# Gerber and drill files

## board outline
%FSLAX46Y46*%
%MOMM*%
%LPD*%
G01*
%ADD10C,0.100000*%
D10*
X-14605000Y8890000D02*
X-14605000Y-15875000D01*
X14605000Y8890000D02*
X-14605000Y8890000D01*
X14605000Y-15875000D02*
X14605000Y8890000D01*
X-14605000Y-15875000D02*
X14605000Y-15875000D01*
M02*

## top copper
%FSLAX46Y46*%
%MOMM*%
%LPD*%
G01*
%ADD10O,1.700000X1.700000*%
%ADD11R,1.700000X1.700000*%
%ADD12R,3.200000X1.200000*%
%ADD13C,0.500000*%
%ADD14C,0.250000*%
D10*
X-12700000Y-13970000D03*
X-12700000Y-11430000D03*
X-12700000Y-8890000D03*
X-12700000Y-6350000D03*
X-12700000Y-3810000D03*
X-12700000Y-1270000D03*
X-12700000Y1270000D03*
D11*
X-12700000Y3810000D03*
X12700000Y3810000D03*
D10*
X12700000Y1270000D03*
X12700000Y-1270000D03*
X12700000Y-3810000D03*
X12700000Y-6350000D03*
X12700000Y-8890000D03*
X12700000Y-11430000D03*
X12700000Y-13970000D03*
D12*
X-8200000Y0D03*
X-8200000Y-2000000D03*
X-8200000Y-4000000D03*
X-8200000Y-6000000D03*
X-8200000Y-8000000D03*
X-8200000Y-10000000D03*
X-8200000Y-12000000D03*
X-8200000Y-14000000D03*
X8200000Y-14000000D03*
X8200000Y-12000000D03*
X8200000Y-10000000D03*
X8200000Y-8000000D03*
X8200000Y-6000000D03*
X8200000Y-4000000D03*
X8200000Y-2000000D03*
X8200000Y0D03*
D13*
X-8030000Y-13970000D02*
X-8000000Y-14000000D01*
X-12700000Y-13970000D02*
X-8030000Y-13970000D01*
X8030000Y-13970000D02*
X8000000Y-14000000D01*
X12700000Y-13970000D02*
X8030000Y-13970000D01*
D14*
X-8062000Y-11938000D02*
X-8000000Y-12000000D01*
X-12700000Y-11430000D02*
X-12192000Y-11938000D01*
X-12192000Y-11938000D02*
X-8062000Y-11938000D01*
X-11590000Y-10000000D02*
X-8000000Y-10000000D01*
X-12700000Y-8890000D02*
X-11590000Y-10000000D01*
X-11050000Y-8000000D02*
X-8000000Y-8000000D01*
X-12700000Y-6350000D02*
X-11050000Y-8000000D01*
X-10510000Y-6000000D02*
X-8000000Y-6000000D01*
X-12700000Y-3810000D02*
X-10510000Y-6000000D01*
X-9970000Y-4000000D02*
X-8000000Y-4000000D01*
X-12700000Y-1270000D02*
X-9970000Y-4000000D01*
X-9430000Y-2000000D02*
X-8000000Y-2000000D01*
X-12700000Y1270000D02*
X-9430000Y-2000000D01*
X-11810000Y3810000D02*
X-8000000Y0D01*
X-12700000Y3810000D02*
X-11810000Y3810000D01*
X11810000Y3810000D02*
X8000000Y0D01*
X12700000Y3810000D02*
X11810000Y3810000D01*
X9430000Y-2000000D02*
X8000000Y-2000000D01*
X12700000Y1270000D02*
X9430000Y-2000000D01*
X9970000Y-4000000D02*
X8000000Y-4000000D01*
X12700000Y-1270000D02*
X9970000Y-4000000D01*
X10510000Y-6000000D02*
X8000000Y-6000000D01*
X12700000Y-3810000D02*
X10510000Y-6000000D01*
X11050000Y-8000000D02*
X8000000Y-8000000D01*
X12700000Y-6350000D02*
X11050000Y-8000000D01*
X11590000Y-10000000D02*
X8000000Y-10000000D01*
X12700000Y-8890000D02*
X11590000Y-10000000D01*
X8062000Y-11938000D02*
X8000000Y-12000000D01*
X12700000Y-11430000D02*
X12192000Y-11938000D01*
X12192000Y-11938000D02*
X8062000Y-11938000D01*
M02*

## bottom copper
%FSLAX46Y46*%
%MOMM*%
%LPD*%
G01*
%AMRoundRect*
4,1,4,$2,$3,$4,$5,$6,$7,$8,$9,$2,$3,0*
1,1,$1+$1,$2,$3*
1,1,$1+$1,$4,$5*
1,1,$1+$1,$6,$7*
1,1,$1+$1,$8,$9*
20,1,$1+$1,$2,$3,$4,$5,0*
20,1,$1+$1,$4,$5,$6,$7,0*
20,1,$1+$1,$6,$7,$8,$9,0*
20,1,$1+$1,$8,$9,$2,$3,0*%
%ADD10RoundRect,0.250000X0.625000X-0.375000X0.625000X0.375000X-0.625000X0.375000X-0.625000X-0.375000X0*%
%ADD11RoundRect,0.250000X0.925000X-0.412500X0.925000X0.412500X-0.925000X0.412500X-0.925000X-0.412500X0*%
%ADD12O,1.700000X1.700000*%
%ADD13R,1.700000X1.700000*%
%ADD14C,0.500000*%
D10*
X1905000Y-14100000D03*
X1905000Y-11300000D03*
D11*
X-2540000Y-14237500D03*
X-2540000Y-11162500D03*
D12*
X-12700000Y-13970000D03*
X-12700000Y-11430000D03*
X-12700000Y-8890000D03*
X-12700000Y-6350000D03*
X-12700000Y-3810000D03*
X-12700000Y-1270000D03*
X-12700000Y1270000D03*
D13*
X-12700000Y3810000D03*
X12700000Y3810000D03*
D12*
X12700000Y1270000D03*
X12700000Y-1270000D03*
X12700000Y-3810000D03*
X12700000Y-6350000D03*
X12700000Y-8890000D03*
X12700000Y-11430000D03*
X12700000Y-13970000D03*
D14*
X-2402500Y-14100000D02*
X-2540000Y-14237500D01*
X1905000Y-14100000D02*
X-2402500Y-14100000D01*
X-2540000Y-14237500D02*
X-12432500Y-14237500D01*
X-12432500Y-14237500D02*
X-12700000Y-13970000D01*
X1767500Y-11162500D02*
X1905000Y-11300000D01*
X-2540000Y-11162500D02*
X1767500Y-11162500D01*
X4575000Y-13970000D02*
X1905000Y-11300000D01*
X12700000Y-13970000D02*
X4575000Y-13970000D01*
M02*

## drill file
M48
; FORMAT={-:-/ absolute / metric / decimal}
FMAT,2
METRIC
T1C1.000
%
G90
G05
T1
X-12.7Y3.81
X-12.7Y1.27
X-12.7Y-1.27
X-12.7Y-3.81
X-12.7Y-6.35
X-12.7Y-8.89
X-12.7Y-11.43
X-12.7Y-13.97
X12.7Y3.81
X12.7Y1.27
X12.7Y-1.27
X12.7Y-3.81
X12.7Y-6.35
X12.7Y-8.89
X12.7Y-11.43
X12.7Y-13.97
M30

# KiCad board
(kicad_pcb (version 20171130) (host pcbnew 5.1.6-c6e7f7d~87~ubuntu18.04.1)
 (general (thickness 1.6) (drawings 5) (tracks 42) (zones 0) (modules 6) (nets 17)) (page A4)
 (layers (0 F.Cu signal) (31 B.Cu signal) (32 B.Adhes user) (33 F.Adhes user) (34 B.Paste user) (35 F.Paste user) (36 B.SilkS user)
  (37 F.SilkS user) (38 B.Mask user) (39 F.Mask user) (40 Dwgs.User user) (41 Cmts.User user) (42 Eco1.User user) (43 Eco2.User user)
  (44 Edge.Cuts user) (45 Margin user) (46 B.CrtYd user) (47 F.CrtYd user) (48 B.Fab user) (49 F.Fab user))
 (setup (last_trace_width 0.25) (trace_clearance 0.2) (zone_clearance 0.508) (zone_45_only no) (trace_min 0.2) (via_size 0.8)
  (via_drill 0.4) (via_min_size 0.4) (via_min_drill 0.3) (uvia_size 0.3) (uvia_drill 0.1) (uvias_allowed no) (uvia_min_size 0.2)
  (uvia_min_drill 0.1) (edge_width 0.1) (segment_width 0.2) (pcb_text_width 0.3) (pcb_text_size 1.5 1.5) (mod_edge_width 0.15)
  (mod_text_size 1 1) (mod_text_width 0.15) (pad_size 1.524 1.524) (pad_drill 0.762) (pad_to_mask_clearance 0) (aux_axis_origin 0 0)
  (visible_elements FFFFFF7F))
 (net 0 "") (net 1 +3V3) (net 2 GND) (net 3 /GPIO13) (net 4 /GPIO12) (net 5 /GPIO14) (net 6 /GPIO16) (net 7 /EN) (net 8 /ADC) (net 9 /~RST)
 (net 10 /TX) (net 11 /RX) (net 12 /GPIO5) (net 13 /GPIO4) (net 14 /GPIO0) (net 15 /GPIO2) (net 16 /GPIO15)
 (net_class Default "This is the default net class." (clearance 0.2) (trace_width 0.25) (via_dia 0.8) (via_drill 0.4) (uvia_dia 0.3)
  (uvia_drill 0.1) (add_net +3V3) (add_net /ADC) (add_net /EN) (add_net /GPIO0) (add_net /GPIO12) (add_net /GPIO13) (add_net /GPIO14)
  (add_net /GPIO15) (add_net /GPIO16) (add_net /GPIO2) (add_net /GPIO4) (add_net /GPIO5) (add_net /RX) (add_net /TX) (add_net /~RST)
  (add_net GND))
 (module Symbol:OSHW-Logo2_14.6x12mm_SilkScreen (layer B.Cu) (at 0 -2.54 180)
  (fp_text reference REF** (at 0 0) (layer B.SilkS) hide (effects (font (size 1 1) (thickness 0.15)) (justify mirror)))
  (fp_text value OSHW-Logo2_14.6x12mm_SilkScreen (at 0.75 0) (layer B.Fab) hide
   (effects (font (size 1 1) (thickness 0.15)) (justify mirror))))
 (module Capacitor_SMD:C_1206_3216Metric (layer B.Cu) (at 1.905 12.7 90)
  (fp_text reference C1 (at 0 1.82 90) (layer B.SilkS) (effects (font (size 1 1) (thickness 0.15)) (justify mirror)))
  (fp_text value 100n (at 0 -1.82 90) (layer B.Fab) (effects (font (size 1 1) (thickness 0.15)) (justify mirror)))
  (pad 1 smd roundrect (at -1.4 0 90) (size 1.25 1.75) (layers B.Cu B.Paste B.Mask) (roundrect_rratio 0.2) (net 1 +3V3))
  (pad 2 smd roundrect (at 1.4 0 90) (size 1.25 1.75) (layers B.Cu B.Paste B.Mask) (roundrect_rratio 0.2) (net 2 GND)))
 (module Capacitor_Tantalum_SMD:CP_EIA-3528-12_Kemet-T (layer B.Cu) (at -2.54 12.7 90)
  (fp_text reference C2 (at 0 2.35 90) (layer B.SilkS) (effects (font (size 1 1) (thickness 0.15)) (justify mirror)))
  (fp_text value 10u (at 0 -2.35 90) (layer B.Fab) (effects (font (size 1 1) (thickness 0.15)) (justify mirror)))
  (pad 1 smd roundrect (at -1.5375 0 90) (size 1.325 2.35) (layers B.Cu B.Paste B.Mask) (roundrect_rratio 0.188679) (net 1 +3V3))
  (pad 2 smd roundrect (at 1.5375 0 90) (size 1.325 2.35) (layers B.Cu B.Paste B.Mask) (roundrect_rratio 0.188679) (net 2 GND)))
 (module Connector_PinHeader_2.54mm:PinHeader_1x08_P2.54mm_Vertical (layer B.Cu) (at -12.7 -3.81 180)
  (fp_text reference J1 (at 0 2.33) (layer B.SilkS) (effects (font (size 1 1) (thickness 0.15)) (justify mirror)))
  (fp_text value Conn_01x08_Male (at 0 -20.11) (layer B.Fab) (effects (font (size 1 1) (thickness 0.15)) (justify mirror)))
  (pad 8 thru_hole oval (at 0 -17.78 180) (size 1.7 1.7) (drill 1) (layers *.Cu *.Mask) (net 1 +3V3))
  (pad 7 thru_hole oval (at 0 -15.24 180) (size 1.7 1.7) (drill 1) (layers *.Cu *.Mask) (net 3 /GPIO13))
  (pad 6 thru_hole oval (at 0 -12.7 180) (size 1.7 1.7) (drill 1) (layers *.Cu *.Mask) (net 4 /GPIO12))
  (pad 5 thru_hole oval (at 0 -10.16 180) (size 1.7 1.7) (drill 1) (layers *.Cu *.Mask) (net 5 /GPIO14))
  (pad 4 thru_hole oval (at 0 -7.62 180) (size 1.7 1.7) (drill 1) (layers *.Cu *.Mask) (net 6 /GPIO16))
  (pad 3 thru_hole oval (at 0 -5.08 180) (size 1.7 1.7) (drill 1) (layers *.Cu *.Mask) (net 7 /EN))
  (pad 2 thru_hole oval (at 0 -2.54 180) (size 1.7 1.7) (drill 1) (layers *.Cu *.Mask) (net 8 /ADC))
  (pad 1 thru_hole rect (at 0 0 180) (size 1.7 1.7) (drill 1) (layers *.Cu *.Mask) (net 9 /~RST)))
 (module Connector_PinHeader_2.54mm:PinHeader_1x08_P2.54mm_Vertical (layer B.Cu) (at 12.7 -3.81 180)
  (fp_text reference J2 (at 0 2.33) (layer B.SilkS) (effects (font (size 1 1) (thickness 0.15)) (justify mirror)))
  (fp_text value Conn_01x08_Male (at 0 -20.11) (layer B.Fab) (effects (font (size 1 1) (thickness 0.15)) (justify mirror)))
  (pad 1 thru_hole rect (at 0 0 180) (size 1.7 1.7) (drill 1) (layers *.Cu *.Mask) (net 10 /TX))
  (pad 2 thru_hole oval (at 0 -2.54 180) (size 1.7 1.7) (drill 1) (layers *.Cu *.Mask) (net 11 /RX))
  (pad 3 thru_hole oval (at 0 -5.08 180) (size 1.7 1.7) (drill 1) (layers *.Cu *.Mask) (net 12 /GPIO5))
  (pad 4 thru_hole oval (at 0 -7.62 180) (size 1.7 1.7) (drill 1) (layers *.Cu *.Mask) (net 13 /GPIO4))
  (pad 5 thru_hole oval (at 0 -10.16 180) (size 1.7 1.7) (drill 1) (layers *.Cu *.Mask) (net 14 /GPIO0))
  (pad 6 thru_hole oval (at 0 -12.7 180) (size 1.7 1.7) (drill 1) (layers *.Cu *.Mask) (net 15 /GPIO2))
  (pad 7 thru_hole oval (at 0 -15.24 180) (size 1.7 1.7) (drill 1) (layers *.Cu *.Mask) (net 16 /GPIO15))
  (pad 8 thru_hole oval (at 0 -17.78 180) (size 1.7 1.7) (drill 1) (layers *.Cu *.Mask) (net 2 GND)))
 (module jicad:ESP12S (layer F.Cu) (at -8 0)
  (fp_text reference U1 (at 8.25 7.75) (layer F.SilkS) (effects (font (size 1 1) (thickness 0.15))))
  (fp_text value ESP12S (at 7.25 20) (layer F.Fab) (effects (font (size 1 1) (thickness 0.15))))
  (pad 1 smd rect (at 0 0) (size 3.2 1.2) (drill (offset -0.2 0)) (layers F.Cu F.Paste F.Mask) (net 9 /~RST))
  (pad 2 smd rect (at 0 2) (size 3.2 1.2) (drill (offset -0.2 0)) (layers F.Cu F.Paste F.Mask) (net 8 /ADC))
  (pad 3 smd rect (at 0 4) (size 3.2 1.2) (drill (offset -0.2 0)) (layers F.Cu F.Paste F.Mask) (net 7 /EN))
  (pad 4 smd rect (at 0 6) (size 3.2 1.2) (drill (offset -0.2 0)) (layers F.Cu F.Paste F.Mask) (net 6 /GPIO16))
  (pad 5 smd rect (at 0 8) (size 3.2 1.2) (drill (offset -0.2 0)) (layers F.Cu F.Paste F.Mask) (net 5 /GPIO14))
  (pad 6 smd rect (at 0 10) (size 3.2 1.2) (drill (offset -0.2 0)) (layers F.Cu F.Paste F.Mask) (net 4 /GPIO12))
  (pad 7 smd rect (at 0 12) (size 3.2 1.2) (drill (offset -0.2 0)) (layers F.Cu F.Paste F.Mask) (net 3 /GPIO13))
  (pad 8 smd rect (at 0 14) (size 3.2 1.2) (drill (offset -0.2 0)) (layers F.Cu F.Paste F.Mask) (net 1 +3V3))
  (pad 9 smd rect (at 16 14 180) (size 3.2 1.2) (drill (offset -0.2 0)) (layers F.Cu F.Paste F.Mask) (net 2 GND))
  (pad 10 smd rect (at 16 12 180) (size 3.2 1.2) (drill (offset -0.2 0)) (layers F.Cu F.Paste F.Mask) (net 16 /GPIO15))
  (pad 11 smd rect (at 16 10 180) (size 3.2 1.2) (drill (offset -0.2 0)) (layers F.Cu F.Paste F.Mask) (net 15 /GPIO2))
  (pad 12 smd rect (at 16 8 180) (size 3.2 1.2) (drill (offset -0.2 0)) (layers F.Cu F.Paste F.Mask) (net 14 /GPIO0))
  (pad 13 smd rect (at 16 6 180) (size 3.2 1.2) (drill (offset -0.2 0)) (layers F.Cu F.Paste F.Mask) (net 13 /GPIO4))
  (pad 14 smd rect (at 16 4 180) (size 3.2 1.2) (drill (offset -0.2 0)) (layers F.Cu F.Paste F.Mask) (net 12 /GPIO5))
  (pad 15 smd rect (at 16 2 180) (size 3.2 1.2) (drill (offset -0.2 0)) (layers F.Cu F.Paste F.Mask) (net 11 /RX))
  (pad 16 smd rect (at 16 0 180) (size 3.2 1.2) (drill (offset -0.2 0)) (layers F.Cu F.Paste F.Mask) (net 10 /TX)))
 (gr_line (start -14.605 -8.89) (end -14.605 15.875) (layer Edge.Cuts) (width 0.1))
 (gr_line (start 14.605 -8.89) (end -14.605 -8.89) (layer Edge.Cuts) (width 0.1))
 (gr_line (start 14.605 15.875) (end 14.605 -8.89) (layer Edge.Cuts) (width 0.1))
 (gr_line (start -14.605 15.875) (end 14.605 15.875) (layer Edge.Cuts) (width 0.1))
 (segment (start -8.03 13.97) (end -8 14) (width 0.5) (layer F.Cu) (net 1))
 (segment (start -12.7 13.97) (end -8.03 13.97) (width 0.5) (layer F.Cu) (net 1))
 (segment (start -2.4025 14.1) (end -2.54 14.2375) (width 0.5) (layer B.Cu) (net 1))
 (segment (start 1.905 14.1) (end -2.4025 14.1) (width 0.5) (layer B.Cu) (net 1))
 (segment (start -2.54 14.2375) (end -12.4325 14.2375) (width 0.5) (layer B.Cu) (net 1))
 (segment (start -12.4325 14.2375) (end -12.7 13.97) (width 0.5) (layer B.Cu) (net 1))
 (segment (start 8.03 13.97) (end 8 14) (width 0.5) (layer F.Cu) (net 2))
 (segment (start 12.7 13.97) (end 8.03 13.97) (width 0.5) (layer F.Cu) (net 2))
 (segment (start 1.7675 11.1625) (end 1.905 11.3) (width 0.5) (layer B.Cu) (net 2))
 (segment (start -2.54 11.1625) (end 1.7675 11.1625) (width 0.5) (layer B.Cu) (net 2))
 (segment (start 4.575 13.97) (end 1.905 11.3) (width 0.5) (layer B.Cu) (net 2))
 (segment (start 12.7 13.97) (end 4.575 13.97) (width 0.5) (layer B.Cu) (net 2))
 (segment (start -8.062 11.938) (end -8 12) (width 0.25) (layer F.Cu) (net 3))
 (segment (start -12.7 11.43) (end -12.192 11.938) (width 0.25) (layer F.Cu) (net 3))
 (segment (start -12.192 11.938) (end -8.062 11.938) (width 0.25) (layer F.Cu) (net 3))
 (segment (start -11.59 10) (end -8 10) (width 0.25) (layer F.Cu) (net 4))
 (segment (start -12.7 8.89) (end -11.59 10) (width 0.25) (layer F.Cu) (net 4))
 (segment (start -11.05 8) (end -8 8) (width 0.25) (layer F.Cu) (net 5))
 (segment (start -12.7 6.35) (end -11.05 8) (width 0.25) (layer F.Cu) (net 5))
 (segment (start -10.51 6) (end -8 6) (width 0.25) (layer F.Cu) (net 6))
 (segment (start -12.7 3.81) (end -10.51 6) (width 0.25) (layer F.Cu) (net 6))
 (segment (start -9.97 4) (end -8 4) (width 0.25) (layer F.Cu) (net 7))
 (segment (start -12.7 1.27) (end -9.97 4) (width 0.25) (layer F.Cu) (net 7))
 (segment (start -9.43 2) (end -8 2) (width 0.25) (layer F.Cu) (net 8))
 (segment (start -12.7 -1.27) (end -9.43 2) (width 0.25) (layer F.Cu) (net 8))
 (segment (start -11.81 -3.81) (end -8 0) (width 0.25) (layer F.Cu) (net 9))
 (segment (start -12.7 -3.81) (end -11.81 -3.81) (width 0.25) (layer F.Cu) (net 9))
 (segment (start 11.81 -3.81) (end 8 0) (width 0.25) (layer F.Cu) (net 10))
 (segment (start 12.7 -3.81) (end 11.81 -3.81) (width 0.25) (layer F.Cu) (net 10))
 (segment (start 9.43 2) (end 8 2) (width 0.25) (layer F.Cu) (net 11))
 (segment (start 12.7 -1.27) (end 9.43 2) (width 0.25) (layer F.Cu) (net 11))
 (segment (start 9.97 4) (end 8 4) (width 0.25) (layer F.Cu) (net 12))
 (segment (start 12.7 1.27) (end 9.97 4) (width 0.25) (layer F.Cu) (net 12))
 (segment (start 10.51 6) (end 8 6) (width 0.25) (layer F.Cu) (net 13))
 (segment (start 12.7 3.81) (end 10.51 6) (width 0.25) (layer F.Cu) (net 13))
 (segment (start 11.05 8) (end 8 8) (width 0.25) (layer F.Cu) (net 14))
 (segment (start 12.7 6.35) (end 11.05 8) (width 0.25) (layer F.Cu) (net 14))
 (segment (start 11.59 10) (end 8 10) (width 0.25) (layer F.Cu) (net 15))
 (segment (start 12.7 8.89) (end 11.59 10) (width 0.25) (layer F.Cu) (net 15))
 (segment (start 8.062 11.938) (end 8 12) (width 0.25) (layer F.Cu) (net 16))
 (segment (start 12.7 11.43) (end 12.192 11.938) (width 0.25) (layer F.Cu) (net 16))
 (segment (start 12.192 11.938) (end 8.062 11.938) (width 0.25) (layer F.Cu) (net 16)))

